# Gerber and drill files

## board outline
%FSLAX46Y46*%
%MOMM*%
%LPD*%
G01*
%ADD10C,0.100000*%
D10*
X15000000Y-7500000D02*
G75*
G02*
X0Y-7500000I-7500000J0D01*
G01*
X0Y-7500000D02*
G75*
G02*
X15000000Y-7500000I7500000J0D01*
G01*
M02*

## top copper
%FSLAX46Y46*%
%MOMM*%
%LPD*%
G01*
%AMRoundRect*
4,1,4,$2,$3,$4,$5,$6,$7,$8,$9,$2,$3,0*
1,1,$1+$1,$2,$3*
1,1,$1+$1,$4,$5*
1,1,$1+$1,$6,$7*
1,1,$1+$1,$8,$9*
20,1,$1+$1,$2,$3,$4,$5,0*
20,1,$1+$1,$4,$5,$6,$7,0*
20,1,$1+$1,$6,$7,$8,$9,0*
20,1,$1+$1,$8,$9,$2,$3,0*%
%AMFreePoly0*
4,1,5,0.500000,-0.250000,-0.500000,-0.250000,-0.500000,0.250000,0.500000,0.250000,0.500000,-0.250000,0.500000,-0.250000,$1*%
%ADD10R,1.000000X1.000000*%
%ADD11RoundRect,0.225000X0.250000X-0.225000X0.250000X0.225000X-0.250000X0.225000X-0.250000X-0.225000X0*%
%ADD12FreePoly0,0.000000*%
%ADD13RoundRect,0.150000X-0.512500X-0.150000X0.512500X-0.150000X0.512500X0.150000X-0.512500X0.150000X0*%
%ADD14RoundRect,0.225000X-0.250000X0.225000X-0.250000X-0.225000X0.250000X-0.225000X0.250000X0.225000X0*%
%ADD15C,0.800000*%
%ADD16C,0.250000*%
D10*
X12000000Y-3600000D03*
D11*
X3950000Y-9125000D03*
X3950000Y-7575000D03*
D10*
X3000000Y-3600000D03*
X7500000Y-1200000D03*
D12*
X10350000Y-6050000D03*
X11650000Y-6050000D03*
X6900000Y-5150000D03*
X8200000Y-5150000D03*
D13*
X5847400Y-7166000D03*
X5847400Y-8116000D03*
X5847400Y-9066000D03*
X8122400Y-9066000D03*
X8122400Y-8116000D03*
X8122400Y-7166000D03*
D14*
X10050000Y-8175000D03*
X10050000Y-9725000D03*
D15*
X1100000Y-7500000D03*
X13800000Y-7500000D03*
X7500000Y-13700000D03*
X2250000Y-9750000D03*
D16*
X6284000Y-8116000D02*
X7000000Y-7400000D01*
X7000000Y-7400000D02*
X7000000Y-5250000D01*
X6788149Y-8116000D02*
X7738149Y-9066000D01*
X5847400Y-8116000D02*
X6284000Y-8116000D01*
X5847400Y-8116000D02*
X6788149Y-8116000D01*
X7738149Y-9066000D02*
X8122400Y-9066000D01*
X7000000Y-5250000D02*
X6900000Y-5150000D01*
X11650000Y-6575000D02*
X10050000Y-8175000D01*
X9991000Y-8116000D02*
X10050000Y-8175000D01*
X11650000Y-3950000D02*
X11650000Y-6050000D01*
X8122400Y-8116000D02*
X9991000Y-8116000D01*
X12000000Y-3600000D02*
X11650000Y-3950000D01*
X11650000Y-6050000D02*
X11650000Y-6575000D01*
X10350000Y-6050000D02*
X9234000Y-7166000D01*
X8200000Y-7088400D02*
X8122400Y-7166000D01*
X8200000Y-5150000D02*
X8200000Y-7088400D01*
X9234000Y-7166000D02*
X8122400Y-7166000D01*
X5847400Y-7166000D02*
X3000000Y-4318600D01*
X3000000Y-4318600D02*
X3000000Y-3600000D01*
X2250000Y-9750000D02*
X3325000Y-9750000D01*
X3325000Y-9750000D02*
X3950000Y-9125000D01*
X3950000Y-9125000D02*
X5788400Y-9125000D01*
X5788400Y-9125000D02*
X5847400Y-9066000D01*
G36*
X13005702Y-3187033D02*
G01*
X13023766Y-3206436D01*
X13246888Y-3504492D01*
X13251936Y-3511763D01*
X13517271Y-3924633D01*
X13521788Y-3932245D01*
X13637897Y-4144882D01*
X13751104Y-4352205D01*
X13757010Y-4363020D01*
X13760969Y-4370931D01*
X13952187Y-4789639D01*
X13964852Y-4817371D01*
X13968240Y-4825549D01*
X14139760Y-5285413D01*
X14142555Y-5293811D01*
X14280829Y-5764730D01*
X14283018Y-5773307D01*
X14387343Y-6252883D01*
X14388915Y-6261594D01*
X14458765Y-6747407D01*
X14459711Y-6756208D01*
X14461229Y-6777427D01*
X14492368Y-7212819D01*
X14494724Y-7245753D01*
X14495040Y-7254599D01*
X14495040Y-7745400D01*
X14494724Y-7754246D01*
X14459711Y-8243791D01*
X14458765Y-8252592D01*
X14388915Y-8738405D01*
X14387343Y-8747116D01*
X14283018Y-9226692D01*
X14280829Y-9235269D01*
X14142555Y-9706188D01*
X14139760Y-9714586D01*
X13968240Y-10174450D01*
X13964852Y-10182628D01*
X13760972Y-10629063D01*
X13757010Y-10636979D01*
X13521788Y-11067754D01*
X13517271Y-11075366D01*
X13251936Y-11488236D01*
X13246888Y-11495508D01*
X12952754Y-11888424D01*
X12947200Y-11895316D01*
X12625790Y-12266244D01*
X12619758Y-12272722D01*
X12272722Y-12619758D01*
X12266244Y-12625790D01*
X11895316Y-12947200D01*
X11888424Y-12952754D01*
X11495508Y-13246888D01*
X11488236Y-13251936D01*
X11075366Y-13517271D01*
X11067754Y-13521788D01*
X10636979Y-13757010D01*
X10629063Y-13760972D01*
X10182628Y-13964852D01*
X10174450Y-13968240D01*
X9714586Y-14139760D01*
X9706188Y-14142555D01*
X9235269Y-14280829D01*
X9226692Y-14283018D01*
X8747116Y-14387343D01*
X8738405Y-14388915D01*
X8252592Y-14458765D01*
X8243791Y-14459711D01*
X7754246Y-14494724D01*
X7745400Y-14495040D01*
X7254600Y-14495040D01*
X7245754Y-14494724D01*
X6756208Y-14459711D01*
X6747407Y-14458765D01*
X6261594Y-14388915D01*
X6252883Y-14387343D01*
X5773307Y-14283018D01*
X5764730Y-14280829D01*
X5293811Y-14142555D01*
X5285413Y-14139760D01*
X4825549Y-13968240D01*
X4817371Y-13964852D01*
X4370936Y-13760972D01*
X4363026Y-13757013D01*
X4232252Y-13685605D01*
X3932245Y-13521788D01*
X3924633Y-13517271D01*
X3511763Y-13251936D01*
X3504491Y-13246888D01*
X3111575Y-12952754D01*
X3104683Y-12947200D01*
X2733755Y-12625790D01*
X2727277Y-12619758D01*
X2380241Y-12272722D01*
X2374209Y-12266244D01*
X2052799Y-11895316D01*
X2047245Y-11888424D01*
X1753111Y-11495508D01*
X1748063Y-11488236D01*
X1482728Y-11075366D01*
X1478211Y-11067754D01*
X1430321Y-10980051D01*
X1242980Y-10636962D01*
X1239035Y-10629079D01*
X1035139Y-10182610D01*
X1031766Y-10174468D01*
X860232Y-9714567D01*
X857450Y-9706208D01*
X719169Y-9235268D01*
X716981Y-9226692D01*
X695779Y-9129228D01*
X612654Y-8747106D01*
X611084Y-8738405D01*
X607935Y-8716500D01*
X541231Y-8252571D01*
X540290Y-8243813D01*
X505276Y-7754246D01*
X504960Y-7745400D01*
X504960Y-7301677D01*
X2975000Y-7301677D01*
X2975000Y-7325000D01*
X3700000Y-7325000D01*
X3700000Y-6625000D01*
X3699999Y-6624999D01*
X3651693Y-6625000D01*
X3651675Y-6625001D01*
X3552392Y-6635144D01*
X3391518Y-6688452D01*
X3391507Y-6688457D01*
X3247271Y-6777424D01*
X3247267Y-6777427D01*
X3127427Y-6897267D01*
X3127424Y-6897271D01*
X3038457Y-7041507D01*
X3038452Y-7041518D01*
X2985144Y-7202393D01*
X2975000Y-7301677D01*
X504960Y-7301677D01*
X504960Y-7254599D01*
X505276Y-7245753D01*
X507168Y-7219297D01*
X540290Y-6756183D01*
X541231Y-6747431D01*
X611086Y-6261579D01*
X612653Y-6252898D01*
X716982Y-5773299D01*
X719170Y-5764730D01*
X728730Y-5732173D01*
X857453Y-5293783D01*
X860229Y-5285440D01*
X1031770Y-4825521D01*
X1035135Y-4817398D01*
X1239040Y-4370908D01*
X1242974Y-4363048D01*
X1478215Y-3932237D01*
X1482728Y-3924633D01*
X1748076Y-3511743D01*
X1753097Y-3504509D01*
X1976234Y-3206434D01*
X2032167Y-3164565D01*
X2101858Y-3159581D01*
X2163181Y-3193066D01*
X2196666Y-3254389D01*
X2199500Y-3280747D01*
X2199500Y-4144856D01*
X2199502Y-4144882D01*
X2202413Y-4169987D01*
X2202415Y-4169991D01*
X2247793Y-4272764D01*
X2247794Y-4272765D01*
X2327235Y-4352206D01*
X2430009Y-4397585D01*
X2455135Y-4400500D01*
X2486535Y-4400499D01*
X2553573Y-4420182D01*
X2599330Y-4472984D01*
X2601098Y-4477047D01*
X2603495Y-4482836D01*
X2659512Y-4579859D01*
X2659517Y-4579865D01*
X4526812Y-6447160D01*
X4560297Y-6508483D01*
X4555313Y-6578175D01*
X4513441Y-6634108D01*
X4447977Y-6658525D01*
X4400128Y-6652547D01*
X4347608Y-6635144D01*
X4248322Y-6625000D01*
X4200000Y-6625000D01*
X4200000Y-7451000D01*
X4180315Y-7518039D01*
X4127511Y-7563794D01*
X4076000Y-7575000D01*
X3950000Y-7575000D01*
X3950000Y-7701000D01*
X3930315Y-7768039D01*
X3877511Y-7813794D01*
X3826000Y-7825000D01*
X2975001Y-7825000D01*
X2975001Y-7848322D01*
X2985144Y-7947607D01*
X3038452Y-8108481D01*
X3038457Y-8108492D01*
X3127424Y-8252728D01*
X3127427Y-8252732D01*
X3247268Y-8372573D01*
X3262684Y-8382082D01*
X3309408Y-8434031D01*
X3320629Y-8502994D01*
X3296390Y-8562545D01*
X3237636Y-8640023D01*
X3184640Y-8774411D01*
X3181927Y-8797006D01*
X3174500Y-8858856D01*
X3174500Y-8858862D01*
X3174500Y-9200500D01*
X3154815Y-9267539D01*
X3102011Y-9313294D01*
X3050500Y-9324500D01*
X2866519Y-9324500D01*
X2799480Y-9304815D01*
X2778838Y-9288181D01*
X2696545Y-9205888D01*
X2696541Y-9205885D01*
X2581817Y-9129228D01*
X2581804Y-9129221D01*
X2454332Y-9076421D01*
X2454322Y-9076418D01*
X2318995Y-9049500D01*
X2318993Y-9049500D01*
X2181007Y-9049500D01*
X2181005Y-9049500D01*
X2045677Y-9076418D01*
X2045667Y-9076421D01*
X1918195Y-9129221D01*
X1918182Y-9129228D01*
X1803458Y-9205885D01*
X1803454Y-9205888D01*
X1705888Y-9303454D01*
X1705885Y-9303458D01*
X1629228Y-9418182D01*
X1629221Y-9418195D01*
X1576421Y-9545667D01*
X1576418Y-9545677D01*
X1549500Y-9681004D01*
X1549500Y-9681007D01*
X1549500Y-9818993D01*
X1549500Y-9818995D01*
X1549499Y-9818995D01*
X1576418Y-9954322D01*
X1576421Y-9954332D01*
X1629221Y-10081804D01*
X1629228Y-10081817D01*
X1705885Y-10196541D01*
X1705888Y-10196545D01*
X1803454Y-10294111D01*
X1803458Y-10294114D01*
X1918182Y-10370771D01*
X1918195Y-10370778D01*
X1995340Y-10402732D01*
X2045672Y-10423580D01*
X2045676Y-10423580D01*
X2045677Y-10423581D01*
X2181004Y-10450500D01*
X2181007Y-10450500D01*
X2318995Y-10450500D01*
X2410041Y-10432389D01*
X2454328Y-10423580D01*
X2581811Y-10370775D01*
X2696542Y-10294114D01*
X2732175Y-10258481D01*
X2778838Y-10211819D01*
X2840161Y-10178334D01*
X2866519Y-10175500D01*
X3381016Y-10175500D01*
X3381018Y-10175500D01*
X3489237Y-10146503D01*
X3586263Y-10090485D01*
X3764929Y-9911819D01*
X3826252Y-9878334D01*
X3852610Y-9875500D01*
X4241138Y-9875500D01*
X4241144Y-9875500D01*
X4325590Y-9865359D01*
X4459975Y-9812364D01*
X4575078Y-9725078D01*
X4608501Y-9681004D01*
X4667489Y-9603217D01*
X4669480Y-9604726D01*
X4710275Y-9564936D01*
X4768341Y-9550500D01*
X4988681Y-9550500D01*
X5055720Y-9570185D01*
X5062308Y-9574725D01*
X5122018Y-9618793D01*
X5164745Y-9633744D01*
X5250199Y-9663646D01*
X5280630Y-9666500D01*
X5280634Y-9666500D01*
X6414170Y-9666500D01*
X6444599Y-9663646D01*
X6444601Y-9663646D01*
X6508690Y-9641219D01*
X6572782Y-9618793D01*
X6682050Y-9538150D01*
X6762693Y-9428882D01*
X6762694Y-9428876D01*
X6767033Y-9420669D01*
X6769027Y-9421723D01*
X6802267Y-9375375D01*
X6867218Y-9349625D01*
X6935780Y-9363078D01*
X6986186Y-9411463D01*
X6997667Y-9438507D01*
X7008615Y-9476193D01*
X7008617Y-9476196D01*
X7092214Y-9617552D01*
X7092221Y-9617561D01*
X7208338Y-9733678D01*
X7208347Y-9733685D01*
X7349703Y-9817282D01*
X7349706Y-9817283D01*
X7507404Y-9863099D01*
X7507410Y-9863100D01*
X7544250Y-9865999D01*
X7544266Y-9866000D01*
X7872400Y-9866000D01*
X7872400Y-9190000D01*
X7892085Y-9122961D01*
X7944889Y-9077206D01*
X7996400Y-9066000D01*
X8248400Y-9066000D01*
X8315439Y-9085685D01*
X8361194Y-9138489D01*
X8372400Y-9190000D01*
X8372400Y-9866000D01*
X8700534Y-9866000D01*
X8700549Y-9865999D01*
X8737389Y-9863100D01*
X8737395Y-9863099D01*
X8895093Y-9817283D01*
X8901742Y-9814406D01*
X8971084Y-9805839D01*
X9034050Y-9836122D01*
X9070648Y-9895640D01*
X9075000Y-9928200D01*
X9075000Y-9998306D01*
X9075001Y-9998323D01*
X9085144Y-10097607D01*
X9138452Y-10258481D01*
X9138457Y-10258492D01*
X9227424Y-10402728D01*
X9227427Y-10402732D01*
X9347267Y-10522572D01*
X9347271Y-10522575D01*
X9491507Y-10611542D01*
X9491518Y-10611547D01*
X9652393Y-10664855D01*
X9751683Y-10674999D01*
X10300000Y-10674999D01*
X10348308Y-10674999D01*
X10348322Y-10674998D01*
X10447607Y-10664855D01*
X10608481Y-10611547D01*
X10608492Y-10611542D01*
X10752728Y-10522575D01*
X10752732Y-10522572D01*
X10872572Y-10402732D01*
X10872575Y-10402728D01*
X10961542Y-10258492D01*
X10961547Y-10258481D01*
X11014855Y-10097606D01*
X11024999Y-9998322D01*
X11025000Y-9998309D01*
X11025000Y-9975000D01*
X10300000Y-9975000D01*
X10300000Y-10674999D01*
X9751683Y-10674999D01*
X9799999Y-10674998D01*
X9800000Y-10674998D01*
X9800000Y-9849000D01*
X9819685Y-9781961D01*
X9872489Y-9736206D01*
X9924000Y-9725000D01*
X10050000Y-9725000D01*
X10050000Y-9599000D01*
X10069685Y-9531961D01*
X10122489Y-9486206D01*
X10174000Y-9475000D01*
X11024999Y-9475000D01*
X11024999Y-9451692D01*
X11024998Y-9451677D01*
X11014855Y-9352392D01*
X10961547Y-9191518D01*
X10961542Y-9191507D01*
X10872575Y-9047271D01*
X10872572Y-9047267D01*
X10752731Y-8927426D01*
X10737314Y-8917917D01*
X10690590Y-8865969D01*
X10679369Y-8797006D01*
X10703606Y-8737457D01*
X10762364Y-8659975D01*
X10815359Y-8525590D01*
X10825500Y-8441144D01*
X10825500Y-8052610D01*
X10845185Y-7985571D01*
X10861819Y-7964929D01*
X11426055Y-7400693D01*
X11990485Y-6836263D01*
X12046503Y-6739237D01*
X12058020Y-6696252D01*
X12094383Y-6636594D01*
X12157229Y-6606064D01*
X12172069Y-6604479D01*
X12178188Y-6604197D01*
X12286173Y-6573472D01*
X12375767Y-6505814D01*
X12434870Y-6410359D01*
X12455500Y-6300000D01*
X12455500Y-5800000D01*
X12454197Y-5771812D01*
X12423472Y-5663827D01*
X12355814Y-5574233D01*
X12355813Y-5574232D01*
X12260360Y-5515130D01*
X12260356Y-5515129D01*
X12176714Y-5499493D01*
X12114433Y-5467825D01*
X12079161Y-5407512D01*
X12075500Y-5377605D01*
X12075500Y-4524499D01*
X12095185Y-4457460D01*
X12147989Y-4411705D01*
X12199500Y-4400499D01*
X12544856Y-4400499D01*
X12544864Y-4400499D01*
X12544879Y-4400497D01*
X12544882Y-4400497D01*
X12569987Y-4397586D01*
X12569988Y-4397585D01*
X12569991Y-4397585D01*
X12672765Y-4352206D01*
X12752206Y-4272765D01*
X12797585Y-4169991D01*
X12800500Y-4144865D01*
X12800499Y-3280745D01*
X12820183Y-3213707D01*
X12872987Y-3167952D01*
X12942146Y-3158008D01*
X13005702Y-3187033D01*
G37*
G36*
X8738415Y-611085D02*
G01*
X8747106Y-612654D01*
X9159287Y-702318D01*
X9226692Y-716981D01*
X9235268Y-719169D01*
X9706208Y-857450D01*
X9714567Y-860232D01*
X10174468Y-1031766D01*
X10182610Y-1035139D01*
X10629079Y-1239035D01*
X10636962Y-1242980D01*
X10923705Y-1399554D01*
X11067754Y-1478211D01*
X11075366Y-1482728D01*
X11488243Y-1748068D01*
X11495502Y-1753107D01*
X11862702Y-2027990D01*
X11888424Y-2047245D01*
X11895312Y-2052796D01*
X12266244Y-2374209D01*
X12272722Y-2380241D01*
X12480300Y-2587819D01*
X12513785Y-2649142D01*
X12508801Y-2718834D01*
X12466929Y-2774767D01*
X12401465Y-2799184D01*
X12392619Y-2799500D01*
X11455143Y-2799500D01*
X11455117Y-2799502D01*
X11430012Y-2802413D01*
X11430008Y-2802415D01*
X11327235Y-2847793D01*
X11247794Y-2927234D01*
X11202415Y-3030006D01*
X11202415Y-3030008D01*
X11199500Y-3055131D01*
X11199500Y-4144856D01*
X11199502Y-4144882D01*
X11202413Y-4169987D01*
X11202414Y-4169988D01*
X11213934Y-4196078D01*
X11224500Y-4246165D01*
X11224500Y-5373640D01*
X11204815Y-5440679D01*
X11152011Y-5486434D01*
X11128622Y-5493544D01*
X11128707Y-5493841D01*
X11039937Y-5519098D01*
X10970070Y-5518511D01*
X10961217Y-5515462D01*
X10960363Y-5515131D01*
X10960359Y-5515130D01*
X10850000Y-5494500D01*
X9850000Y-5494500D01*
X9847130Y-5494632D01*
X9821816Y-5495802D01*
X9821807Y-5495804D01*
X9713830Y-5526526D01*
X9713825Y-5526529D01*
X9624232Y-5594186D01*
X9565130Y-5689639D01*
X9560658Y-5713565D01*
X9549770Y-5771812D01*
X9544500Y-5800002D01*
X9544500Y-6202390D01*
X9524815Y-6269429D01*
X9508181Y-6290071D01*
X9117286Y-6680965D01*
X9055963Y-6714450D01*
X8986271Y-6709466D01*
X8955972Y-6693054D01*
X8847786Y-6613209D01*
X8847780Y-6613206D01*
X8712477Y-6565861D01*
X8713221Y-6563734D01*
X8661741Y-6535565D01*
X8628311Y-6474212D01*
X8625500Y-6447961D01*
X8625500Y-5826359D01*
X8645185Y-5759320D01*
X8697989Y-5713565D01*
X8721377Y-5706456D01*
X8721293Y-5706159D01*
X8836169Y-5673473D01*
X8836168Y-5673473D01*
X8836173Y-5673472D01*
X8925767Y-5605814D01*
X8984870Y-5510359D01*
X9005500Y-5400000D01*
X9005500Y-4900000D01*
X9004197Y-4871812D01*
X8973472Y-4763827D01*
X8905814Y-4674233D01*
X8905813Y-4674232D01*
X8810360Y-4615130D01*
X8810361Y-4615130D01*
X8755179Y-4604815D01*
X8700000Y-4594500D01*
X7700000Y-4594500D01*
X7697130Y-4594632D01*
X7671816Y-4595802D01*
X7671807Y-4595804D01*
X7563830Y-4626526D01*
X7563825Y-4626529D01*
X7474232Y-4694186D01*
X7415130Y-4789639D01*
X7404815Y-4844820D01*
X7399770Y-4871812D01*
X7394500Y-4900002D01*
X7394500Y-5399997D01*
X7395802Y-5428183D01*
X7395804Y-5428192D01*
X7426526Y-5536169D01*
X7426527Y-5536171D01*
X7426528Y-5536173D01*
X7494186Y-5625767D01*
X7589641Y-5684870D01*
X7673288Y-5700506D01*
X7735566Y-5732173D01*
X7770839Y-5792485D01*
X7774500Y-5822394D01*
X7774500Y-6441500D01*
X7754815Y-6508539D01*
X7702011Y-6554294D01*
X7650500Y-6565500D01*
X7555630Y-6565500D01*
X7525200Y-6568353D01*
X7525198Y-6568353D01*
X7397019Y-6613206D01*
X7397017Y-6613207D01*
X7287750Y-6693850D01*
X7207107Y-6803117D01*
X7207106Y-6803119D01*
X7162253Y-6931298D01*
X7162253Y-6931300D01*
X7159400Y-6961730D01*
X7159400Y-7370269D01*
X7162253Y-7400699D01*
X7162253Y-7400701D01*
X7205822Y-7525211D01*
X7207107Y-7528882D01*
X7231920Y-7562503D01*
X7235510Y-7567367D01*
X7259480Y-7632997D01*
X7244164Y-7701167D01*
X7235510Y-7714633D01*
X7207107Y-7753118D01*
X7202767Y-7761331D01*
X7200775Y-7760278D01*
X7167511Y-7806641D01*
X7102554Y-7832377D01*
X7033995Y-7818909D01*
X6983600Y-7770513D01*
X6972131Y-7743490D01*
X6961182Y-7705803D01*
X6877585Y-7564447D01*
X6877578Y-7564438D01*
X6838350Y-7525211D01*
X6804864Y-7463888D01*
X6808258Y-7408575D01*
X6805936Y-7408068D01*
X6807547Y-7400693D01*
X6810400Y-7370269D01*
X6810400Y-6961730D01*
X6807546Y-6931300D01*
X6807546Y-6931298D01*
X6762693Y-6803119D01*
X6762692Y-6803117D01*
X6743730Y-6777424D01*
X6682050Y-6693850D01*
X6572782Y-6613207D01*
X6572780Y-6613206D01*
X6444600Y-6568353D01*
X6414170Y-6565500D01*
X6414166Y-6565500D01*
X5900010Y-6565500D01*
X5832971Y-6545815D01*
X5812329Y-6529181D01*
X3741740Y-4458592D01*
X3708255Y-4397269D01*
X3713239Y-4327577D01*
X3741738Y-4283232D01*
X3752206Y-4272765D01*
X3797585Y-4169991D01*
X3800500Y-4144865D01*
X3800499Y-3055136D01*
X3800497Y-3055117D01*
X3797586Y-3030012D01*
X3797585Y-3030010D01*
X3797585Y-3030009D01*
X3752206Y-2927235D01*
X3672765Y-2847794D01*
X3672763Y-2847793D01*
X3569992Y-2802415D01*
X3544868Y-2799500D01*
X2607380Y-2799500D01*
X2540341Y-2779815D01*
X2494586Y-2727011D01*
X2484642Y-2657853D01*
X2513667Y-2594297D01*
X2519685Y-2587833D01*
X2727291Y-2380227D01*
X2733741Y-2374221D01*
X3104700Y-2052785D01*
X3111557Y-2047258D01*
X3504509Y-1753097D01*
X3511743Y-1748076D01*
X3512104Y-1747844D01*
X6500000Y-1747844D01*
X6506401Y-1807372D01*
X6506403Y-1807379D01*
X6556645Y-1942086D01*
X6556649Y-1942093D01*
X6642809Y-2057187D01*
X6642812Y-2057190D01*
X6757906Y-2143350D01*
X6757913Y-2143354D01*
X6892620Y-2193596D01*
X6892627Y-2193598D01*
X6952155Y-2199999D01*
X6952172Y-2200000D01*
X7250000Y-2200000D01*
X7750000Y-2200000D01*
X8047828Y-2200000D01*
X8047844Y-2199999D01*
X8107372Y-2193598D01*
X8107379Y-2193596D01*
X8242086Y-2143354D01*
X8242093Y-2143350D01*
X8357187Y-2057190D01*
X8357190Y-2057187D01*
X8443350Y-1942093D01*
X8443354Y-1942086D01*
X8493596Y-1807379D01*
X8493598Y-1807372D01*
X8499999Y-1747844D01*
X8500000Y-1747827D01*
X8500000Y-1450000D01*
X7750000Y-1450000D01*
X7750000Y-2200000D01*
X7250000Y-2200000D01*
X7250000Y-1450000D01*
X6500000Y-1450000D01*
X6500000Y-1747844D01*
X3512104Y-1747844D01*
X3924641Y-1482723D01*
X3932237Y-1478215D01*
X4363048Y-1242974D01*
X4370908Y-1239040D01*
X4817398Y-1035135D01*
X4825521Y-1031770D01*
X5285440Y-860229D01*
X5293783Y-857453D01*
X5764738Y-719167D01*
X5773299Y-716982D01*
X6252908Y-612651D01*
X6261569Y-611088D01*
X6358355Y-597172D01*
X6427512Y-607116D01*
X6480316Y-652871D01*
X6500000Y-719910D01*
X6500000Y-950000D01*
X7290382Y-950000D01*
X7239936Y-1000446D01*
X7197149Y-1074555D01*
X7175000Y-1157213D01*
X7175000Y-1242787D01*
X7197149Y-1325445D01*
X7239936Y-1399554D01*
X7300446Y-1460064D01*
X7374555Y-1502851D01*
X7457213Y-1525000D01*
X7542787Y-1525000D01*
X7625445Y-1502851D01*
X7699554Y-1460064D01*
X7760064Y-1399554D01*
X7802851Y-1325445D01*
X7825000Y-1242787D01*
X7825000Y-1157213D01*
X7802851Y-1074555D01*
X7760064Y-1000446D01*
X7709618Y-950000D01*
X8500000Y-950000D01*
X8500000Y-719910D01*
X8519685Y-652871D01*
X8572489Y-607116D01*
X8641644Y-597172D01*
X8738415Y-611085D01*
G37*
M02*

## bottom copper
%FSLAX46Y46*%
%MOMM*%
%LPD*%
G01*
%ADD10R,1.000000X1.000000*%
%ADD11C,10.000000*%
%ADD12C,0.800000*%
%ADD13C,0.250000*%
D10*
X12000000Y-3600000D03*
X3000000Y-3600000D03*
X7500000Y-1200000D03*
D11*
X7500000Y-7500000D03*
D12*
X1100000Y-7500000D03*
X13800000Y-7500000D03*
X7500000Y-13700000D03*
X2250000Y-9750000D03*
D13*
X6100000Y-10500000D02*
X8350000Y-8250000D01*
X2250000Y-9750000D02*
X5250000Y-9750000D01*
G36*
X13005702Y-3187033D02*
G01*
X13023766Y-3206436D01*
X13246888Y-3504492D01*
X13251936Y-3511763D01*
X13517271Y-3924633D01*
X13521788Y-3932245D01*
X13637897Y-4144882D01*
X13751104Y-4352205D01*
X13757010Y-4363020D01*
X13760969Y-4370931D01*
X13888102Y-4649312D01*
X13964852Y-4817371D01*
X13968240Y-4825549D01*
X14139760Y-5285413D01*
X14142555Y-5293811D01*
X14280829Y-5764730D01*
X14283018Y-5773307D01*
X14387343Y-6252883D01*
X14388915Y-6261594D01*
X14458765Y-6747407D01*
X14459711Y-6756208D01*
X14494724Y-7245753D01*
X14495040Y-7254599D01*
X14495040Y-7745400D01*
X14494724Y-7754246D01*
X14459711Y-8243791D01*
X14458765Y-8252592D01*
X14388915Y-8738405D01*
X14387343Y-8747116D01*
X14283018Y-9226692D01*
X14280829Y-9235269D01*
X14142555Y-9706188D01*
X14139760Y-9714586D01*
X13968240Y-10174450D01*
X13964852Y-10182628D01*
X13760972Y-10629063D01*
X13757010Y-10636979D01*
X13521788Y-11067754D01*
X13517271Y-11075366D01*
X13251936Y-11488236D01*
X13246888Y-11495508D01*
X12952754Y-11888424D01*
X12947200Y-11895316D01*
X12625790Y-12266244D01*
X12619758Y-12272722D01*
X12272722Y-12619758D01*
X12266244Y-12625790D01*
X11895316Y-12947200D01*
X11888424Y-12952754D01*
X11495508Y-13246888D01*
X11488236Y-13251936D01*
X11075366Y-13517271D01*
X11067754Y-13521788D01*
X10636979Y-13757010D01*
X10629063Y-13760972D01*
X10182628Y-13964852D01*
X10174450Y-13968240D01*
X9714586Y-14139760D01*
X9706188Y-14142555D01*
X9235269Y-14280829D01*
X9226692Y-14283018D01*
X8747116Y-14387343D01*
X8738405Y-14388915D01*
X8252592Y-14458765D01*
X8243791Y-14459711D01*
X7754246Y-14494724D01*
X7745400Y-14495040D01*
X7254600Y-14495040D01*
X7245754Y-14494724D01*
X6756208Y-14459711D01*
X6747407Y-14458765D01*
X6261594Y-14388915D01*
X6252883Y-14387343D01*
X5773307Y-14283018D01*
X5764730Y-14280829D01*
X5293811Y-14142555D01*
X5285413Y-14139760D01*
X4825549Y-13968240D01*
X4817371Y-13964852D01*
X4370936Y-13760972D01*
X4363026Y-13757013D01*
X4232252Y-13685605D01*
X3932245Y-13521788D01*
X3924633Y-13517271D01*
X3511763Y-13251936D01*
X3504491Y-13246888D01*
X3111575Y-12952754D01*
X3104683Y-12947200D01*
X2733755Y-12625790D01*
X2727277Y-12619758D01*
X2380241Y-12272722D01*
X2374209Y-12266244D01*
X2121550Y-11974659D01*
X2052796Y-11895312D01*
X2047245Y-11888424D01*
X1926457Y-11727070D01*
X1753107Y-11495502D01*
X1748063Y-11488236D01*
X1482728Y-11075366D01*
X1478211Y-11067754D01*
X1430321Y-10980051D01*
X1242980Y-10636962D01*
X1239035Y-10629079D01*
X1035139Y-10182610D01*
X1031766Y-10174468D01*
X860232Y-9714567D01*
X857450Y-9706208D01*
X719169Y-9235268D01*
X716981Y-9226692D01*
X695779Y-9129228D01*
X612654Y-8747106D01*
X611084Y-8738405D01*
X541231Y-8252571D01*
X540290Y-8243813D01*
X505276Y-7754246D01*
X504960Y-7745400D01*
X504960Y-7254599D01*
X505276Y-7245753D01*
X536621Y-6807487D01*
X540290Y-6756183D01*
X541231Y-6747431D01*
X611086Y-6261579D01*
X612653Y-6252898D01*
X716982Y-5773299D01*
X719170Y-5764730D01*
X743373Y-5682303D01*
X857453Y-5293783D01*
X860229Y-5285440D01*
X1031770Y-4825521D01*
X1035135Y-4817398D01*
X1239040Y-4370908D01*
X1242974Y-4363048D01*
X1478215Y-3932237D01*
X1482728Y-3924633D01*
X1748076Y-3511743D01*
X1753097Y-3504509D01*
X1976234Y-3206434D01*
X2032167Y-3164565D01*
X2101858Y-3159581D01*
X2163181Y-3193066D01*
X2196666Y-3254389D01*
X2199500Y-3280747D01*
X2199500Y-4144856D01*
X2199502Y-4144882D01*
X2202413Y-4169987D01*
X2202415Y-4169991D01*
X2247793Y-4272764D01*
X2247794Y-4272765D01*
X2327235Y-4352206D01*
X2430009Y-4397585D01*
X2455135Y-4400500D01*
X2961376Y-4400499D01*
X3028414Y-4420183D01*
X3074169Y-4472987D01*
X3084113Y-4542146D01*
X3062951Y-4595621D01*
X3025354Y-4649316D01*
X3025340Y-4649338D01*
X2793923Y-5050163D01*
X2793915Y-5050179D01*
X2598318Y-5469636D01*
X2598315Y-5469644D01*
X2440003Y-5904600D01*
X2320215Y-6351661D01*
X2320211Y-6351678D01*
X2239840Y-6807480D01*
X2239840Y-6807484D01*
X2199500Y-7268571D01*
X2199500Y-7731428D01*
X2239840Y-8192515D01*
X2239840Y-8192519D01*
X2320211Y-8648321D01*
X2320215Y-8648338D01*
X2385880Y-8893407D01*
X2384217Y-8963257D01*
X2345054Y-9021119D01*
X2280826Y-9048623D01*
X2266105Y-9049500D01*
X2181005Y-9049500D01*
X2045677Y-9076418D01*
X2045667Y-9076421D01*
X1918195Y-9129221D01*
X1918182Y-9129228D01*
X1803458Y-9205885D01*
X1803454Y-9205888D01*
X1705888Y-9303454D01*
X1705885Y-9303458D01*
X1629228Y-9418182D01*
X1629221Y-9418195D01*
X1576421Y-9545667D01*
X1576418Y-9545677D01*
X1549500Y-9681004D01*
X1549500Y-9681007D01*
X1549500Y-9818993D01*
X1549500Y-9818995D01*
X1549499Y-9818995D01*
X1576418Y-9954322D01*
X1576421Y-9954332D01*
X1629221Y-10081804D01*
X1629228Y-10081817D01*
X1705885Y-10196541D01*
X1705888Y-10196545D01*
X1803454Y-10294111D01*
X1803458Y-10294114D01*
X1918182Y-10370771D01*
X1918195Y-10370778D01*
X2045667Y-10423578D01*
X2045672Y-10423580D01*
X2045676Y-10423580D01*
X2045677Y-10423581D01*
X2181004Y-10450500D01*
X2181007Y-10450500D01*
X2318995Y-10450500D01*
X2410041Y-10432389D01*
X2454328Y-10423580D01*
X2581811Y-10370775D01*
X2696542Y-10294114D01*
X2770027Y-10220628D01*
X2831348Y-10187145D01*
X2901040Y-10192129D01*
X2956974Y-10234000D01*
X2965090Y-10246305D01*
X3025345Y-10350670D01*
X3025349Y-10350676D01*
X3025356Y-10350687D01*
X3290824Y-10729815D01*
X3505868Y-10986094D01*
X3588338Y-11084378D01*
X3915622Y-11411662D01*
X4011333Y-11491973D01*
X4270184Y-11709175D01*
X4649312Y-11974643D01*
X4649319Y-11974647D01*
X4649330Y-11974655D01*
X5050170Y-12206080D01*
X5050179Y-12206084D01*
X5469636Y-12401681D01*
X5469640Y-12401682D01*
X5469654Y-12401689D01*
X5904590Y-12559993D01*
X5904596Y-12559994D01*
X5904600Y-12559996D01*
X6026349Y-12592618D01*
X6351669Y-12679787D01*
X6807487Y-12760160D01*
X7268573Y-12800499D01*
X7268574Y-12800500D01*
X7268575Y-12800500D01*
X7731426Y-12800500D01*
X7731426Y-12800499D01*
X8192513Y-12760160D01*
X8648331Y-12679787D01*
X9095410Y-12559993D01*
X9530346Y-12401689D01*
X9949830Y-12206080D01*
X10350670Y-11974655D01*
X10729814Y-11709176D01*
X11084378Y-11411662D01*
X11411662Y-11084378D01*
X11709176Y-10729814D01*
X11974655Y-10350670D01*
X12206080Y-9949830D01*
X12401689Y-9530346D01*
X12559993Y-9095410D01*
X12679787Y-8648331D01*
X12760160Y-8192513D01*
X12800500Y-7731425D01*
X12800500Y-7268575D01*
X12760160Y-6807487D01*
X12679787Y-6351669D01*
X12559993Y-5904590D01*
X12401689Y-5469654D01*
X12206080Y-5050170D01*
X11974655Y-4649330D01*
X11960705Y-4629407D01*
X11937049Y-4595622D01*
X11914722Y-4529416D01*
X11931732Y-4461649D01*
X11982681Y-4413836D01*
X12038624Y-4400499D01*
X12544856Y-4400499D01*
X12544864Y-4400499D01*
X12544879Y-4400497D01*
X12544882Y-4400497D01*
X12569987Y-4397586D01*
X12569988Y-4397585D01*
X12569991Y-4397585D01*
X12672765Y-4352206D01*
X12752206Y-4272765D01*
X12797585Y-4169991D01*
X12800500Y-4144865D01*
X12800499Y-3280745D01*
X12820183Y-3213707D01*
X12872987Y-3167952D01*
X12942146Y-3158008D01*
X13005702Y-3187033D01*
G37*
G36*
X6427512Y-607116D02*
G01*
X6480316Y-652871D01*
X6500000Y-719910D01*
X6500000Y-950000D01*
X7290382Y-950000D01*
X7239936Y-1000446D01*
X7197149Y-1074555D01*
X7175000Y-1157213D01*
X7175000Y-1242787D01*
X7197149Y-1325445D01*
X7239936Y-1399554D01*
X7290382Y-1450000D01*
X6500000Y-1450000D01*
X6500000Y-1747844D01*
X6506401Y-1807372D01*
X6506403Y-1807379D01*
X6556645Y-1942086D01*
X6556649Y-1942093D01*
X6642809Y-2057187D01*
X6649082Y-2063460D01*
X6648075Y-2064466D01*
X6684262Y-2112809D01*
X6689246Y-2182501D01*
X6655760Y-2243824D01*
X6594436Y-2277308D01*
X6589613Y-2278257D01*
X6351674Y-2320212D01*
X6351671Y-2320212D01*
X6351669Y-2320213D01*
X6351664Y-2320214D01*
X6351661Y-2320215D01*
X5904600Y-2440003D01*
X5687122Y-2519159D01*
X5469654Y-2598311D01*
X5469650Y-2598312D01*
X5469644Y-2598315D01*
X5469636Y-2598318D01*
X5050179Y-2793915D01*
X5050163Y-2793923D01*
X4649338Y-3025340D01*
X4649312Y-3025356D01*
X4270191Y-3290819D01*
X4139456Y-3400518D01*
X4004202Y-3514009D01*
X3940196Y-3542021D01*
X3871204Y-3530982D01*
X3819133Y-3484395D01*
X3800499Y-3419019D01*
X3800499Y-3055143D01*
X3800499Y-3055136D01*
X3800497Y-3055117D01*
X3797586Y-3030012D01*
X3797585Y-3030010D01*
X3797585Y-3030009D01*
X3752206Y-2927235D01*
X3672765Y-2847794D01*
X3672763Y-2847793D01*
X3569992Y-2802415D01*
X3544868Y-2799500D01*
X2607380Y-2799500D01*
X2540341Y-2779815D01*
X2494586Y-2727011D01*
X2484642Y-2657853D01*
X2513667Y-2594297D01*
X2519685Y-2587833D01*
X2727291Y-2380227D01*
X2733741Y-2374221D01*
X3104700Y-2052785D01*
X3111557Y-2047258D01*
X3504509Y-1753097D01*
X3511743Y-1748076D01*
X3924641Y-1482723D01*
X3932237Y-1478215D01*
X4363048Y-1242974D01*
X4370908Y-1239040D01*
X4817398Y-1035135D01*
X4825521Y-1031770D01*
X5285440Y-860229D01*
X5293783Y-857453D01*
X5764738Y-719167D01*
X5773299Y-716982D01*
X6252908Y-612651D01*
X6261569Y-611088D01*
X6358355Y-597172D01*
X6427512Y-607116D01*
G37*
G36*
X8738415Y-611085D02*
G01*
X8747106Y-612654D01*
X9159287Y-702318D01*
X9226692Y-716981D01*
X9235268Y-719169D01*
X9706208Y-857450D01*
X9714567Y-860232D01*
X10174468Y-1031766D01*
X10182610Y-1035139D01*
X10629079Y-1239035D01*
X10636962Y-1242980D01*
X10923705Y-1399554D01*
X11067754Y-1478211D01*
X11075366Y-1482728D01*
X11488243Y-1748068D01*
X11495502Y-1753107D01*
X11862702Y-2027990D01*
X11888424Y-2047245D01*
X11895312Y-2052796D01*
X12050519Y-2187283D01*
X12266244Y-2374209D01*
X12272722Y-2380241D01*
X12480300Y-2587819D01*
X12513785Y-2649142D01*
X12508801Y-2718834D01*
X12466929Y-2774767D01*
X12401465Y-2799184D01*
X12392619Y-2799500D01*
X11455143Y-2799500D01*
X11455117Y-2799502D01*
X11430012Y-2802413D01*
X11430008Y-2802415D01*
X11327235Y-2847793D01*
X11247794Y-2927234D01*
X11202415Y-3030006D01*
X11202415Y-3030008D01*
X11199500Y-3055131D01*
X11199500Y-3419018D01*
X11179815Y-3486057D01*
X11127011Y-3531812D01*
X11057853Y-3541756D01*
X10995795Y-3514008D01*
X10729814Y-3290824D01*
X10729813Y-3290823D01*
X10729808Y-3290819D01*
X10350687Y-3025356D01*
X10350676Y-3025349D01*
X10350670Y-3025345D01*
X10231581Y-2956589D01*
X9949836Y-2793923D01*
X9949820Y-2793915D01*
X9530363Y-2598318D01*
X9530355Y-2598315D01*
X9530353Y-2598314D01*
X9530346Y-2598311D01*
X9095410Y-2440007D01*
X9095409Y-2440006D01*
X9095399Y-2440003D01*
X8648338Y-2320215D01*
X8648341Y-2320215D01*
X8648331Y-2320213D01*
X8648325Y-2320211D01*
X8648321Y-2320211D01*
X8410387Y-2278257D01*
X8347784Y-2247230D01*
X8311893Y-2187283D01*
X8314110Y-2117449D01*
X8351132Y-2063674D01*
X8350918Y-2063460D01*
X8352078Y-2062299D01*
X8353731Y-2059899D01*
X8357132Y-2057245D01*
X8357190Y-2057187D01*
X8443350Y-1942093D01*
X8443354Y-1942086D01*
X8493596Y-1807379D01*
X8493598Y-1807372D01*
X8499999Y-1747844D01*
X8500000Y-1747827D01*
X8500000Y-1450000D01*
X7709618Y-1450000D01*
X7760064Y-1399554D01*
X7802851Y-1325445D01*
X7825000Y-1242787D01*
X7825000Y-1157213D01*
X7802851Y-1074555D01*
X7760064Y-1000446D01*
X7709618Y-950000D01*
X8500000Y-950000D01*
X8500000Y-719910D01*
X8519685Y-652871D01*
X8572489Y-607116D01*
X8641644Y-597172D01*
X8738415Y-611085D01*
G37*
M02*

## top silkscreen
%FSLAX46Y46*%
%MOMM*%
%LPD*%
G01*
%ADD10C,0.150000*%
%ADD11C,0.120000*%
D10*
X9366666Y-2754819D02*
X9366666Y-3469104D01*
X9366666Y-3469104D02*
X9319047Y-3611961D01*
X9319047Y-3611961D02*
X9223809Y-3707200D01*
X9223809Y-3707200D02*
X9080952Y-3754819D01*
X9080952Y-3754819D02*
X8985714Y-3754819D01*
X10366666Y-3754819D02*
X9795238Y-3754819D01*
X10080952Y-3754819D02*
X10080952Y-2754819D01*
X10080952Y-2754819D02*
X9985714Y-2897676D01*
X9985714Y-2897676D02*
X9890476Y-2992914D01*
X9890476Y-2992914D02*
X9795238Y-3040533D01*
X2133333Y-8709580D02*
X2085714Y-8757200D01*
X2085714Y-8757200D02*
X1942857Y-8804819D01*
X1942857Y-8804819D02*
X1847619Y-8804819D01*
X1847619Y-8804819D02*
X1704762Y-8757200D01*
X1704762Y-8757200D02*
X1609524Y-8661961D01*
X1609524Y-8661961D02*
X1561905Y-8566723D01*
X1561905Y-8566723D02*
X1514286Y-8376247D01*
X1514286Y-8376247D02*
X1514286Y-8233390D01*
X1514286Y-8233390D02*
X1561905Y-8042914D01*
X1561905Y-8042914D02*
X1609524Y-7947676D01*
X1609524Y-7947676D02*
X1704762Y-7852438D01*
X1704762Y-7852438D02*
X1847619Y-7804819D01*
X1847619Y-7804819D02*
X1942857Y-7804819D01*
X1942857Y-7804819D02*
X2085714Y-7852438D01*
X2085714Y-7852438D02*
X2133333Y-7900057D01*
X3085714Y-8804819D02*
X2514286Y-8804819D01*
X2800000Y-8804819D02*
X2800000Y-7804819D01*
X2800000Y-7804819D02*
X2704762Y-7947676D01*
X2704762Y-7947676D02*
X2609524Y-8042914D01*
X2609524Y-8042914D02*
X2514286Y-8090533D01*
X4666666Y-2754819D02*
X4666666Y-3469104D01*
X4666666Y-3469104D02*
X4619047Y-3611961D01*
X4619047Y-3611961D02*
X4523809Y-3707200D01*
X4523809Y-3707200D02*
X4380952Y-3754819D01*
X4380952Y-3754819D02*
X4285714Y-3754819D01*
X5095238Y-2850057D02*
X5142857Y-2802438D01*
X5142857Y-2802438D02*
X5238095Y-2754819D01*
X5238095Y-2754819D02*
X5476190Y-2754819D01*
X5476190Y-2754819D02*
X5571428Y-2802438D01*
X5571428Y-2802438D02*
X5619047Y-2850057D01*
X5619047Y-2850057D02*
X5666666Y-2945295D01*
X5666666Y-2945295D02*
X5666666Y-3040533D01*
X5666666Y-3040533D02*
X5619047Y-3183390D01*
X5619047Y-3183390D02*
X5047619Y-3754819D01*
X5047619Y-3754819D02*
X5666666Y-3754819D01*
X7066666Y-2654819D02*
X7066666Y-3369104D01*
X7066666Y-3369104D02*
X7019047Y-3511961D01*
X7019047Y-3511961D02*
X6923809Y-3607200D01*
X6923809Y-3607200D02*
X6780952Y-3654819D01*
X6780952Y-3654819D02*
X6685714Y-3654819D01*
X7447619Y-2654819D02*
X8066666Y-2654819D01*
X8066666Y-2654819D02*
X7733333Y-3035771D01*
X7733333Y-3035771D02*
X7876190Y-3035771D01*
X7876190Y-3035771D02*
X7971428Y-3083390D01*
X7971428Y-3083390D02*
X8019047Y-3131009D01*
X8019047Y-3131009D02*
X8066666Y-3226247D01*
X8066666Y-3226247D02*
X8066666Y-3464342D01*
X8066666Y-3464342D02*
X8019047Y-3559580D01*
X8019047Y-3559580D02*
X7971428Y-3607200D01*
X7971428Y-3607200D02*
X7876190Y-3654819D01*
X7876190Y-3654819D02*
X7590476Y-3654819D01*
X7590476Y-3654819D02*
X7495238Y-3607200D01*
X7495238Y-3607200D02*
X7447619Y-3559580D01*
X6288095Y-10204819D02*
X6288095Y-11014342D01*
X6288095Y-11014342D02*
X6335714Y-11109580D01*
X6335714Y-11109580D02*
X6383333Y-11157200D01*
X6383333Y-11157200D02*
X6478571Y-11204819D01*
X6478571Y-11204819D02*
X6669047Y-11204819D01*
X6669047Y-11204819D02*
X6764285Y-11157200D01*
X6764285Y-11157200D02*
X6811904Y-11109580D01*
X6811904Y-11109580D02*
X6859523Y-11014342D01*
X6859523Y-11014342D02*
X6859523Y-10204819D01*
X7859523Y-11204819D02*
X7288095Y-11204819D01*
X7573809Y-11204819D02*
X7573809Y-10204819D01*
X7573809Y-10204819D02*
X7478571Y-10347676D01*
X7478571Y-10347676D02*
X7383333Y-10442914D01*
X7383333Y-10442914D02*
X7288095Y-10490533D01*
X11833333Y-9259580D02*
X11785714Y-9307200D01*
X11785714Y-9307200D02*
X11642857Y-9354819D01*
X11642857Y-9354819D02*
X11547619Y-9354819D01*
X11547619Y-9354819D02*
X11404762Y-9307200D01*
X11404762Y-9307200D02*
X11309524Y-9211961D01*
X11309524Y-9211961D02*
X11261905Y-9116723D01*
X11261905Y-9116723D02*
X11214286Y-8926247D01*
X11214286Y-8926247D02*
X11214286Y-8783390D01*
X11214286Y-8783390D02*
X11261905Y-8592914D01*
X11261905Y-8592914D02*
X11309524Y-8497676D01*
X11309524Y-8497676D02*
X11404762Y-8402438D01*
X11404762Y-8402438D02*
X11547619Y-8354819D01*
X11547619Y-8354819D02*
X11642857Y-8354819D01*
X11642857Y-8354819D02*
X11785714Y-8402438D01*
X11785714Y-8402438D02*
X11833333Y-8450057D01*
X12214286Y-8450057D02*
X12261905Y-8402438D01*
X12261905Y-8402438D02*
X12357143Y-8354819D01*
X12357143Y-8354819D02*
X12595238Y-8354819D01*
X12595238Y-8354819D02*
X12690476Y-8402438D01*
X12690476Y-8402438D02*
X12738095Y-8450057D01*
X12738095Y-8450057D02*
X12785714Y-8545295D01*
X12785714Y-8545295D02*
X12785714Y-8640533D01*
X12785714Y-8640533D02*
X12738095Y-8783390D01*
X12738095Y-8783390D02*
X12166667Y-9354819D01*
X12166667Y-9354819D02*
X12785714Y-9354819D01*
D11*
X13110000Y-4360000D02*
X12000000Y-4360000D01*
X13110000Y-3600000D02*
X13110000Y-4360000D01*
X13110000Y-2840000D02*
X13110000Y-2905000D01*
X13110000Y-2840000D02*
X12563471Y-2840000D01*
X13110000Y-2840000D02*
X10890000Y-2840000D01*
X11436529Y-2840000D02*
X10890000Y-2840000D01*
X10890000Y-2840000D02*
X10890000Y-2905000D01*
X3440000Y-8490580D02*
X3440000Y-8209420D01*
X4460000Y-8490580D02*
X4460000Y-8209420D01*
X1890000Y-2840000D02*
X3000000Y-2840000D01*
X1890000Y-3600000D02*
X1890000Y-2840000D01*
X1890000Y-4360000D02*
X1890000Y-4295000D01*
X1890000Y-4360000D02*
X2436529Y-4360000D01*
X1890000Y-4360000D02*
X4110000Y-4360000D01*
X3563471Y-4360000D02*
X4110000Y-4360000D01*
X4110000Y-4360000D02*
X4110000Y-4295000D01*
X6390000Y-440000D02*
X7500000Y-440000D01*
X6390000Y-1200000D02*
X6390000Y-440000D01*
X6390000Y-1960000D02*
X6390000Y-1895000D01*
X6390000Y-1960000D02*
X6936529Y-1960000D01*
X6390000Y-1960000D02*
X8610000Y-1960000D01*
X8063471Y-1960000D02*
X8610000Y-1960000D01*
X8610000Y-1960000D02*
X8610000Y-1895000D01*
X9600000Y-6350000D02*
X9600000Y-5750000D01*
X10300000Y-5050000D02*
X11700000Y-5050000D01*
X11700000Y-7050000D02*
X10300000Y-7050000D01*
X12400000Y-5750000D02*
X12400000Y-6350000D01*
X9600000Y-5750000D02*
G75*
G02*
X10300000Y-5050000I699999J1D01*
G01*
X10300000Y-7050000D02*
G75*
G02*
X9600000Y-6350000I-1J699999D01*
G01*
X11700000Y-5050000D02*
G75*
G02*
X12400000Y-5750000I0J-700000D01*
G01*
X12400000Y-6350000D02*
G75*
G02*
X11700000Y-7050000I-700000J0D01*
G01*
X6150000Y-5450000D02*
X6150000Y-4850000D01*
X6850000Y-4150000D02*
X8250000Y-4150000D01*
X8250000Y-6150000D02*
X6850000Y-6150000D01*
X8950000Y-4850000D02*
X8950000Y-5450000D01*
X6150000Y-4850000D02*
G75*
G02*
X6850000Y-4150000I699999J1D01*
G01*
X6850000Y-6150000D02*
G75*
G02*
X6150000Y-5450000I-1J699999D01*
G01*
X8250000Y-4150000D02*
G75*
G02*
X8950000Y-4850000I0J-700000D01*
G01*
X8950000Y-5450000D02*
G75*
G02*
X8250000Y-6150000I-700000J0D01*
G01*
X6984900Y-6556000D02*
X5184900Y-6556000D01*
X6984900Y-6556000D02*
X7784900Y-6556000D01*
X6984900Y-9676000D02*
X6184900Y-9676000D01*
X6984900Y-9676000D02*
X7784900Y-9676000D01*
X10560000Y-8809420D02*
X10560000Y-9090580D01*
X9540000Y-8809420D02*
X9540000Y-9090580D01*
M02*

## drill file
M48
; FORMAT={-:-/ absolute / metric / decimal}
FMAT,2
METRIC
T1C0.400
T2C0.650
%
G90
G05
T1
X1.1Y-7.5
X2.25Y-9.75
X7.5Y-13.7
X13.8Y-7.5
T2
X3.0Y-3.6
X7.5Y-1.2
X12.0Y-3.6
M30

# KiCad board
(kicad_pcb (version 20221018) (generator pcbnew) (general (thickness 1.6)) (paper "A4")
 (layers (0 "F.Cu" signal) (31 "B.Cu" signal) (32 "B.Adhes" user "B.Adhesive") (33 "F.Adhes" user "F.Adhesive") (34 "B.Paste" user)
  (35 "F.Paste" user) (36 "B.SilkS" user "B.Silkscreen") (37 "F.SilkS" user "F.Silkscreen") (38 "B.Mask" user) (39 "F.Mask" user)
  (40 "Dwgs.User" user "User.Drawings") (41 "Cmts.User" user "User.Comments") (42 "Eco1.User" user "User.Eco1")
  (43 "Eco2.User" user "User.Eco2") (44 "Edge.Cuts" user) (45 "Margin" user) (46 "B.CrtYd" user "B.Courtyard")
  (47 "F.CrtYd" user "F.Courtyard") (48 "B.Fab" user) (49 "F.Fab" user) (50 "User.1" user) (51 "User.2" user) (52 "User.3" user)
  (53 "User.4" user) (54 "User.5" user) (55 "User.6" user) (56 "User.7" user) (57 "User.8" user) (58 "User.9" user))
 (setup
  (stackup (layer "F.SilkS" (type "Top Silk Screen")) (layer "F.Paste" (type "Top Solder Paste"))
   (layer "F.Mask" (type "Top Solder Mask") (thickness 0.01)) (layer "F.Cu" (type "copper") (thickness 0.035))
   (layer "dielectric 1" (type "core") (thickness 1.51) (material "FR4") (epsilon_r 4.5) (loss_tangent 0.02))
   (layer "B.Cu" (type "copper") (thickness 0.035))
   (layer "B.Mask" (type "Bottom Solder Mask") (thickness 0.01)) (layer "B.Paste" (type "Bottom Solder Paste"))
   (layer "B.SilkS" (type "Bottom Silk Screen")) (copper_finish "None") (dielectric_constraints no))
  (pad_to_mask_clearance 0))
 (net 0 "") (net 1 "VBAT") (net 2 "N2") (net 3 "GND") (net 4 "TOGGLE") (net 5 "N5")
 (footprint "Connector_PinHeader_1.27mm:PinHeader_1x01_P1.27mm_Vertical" (layer "F.Cu") (at 12 3.6 180)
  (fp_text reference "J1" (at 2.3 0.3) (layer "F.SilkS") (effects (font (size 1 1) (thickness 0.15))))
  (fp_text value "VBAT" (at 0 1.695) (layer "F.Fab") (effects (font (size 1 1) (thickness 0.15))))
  (fp_line (start -1.11 -0.76) (end 0 -0.76) (stroke (width 0.12) (type solid)) (layer "F.SilkS"))
  (fp_line (start -1.11 0) (end -1.11 -0.76) (stroke (width 0.12) (type solid)) (layer "F.SilkS"))
  (fp_line (start -1.11 0.76) (end -1.11 0.695) (stroke (width 0.12) (type solid)) (layer "F.SilkS"))
  (fp_line (start -1.11 0.76) (end -0.563471 0.76) (stroke (width 0.12) (type solid)) (layer "F.SilkS"))
  (fp_line (start -1.11 0.76) (end 1.11 0.76) (stroke (width 0.12) (type solid)) (layer "F.SilkS"))
  (fp_line (start 0.563471 0.76) (end 1.11 0.76) (stroke (width 0.12) (type solid)) (layer "F.SilkS"))
  (fp_line (start 1.11 0.76) (end 1.11 0.695) (stroke (width 0.12) (type solid)) (layer "F.SilkS"))
  (pad "1" thru_hole rect (at 0 0 180) (size 1 1) (drill 0.65) (layers "*.Cu" "*.Mask") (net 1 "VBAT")))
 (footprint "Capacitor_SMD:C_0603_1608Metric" (layer "F.Cu") (at 3.95 8.35 90)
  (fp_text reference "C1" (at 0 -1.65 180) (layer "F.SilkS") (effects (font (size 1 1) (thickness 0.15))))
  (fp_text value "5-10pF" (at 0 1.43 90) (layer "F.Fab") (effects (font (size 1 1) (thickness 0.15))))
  (fp_line (start -0.14058 -0.51) (end 0.14058 -0.51) (stroke (width 0.12) (type solid)) (layer "F.SilkS"))
  (fp_line (start -0.14058 0.51) (end 0.14058 0.51) (stroke (width 0.12) (type solid)) (layer "F.SilkS"))
  (pad "1" smd roundrect (at -0.775 0 90) (size 0.9 0.95) (layers "F.Cu" "F.Paste" "F.Mask") (roundrect_rratio 0.25) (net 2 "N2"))
  (pad "2" smd roundrect (at 0.775 0 90) (size 0.9 0.95) (layers "F.Cu" "F.Paste" "F.Mask") (roundrect_rratio 0.25) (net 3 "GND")))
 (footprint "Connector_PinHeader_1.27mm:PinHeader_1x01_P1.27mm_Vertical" (layer "F.Cu") (at 3 3.6)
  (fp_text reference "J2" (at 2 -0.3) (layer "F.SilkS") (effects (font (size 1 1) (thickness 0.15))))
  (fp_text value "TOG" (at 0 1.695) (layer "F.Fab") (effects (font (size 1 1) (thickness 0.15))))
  (fp_line (start -1.11 -0.76) (end 0 -0.76) (stroke (width 0.12) (type solid)) (layer "F.SilkS"))
  (fp_line (start -1.11 0) (end -1.11 -0.76) (stroke (width 0.12) (type solid)) (layer "F.SilkS"))
  (fp_line (start -1.11 0.76) (end -1.11 0.695) (stroke (width 0.12) (type solid)) (layer "F.SilkS"))
  (fp_line (start -1.11 0.76) (end -0.563471 0.76) (stroke (width 0.12) (type solid)) (layer "F.SilkS"))
  (fp_line (start -1.11 0.76) (end 1.11 0.76) (stroke (width 0.12) (type solid)) (layer "F.SilkS"))
  (fp_line (start 0.563471 0.76) (end 1.11 0.76) (stroke (width 0.12) (type solid)) (layer "F.SilkS"))
  (fp_line (start 1.11 0.76) (end 1.11 0.695) (stroke (width 0.12) (type solid)) (layer "F.SilkS"))
  (pad "1" thru_hole rect (at 0 0) (size 1 1) (drill 0.65) (layers "*.Cu" "*.Mask") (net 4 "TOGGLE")))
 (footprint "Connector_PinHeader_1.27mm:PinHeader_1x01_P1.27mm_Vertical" (layer "F.Cu") (at 7.5 1.2)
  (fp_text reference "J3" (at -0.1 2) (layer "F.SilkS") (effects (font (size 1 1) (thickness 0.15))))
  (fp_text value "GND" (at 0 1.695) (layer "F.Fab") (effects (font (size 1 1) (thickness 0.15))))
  (fp_line (start -1.11 -0.76) (end 0 -0.76) (stroke (width 0.12) (type solid)) (layer "F.SilkS"))
  (fp_line (start -1.11 0) (end -1.11 -0.76) (stroke (width 0.12) (type solid)) (layer "F.SilkS"))
  (fp_line (start -1.11 0.76) (end -1.11 0.695) (stroke (width 0.12) (type solid)) (layer "F.SilkS"))
  (fp_line (start -1.11 0.76) (end -0.563471 0.76) (stroke (width 0.12) (type solid)) (layer "F.SilkS"))
  (fp_line (start -1.11 0.76) (end 1.11 0.76) (stroke (width 0.12) (type solid)) (layer "F.SilkS"))
  (fp_line (start 0.563471 0.76) (end 1.11 0.76) (stroke (width 0.12) (type solid)) (layer "F.SilkS"))
  (fp_line (start 1.11 0.76) (end 1.11 0.695) (stroke (width 0.12) (type solid)) (layer "F.SilkS"))
  (pad "1" thru_hole rect (at 0 0) (size 1 1) (drill 0.65) (layers "*.Cu" "*.Mask") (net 3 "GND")))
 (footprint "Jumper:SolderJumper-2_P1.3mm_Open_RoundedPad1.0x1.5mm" (layer "F.Cu") (at 11 6.05)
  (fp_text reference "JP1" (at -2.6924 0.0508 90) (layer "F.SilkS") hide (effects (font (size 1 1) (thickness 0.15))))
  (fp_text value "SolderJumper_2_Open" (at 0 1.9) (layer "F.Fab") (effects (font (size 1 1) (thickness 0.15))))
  (fp_line (start -1.4 0.3) (end -1.4 -0.3) (stroke (width 0.12) (type solid)) (layer "F.SilkS"))
  (fp_line (start -0.7 -1) (end 0.7 -1) (stroke (width 0.12) (type solid)) (layer "F.SilkS"))
  (fp_line (start 0.7 1) (end -0.7 1) (stroke (width 0.12) (type solid)) (layer "F.SilkS"))
  (fp_line (start 1.4 -0.3) (end 1.4 0.3) (stroke (width 0.12) (type solid)) (layer "F.SilkS"))
  (fp_arc (start -1.4 -0.3) (mid -1.194975 -0.794975) (end -0.7 -1) (stroke (width 0.12) (type solid)) (layer "F.SilkS"))
  (fp_arc (start -0.7 1) (mid -1.194975 0.794975) (end -1.4 0.3) (stroke (width 0.12) (type solid)) (layer "F.SilkS"))
  (fp_arc (start 0.7 -1) (mid 1.194975 -0.794975) (end 1.4 -0.3) (stroke (width 0.12) (type solid)) (layer "F.SilkS"))
  (fp_arc (start 1.4 0.3) (mid 1.194975 0.794975) (end 0.7 1) (stroke (width 0.12) (type solid)) (layer "F.SilkS"))
  (pad "1" smd custom (at -0.65 0) (size 1 0.5) (layers "F.Cu" "F.Mask") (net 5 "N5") (zone_connect 2) (thermal_bridge_angle 45)
   (options (clearance outline) (anchor rect)) (primitives))
  (pad "2" smd custom (at 0.65 0) (size 1 0.5) (layers "F.Cu" "F.Mask") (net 1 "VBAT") (zone_connect 2) (thermal_bridge_angle 45)
   (options (clearance outline) (anchor rect)) (primitives)))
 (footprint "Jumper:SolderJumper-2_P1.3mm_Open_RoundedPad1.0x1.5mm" (layer "F.Cu") (at 7.55 5.15)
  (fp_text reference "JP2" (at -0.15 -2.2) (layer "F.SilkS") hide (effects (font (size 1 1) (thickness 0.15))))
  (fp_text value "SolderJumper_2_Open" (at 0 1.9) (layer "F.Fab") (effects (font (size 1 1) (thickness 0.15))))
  (fp_line (start -1.4 0.3) (end -1.4 -0.3) (stroke (width 0.12) (type solid)) (layer "F.SilkS"))
  (fp_line (start -0.7 -1) (end 0.7 -1) (stroke (width 0.12) (type solid)) (layer "F.SilkS"))
  (fp_line (start 0.7 1) (end -0.7 1) (stroke (width 0.12) (type solid)) (layer "F.SilkS"))
  (fp_line (start 1.4 -0.3) (end 1.4 0.3) (stroke (width 0.12) (type solid)) (layer "F.SilkS"))
  (fp_arc (start -1.4 -0.3) (mid -1.194975 -0.794975) (end -0.7 -1) (stroke (width 0.12) (type solid)) (layer "F.SilkS"))
  (fp_arc (start -0.7 1) (mid -1.194975 0.794975) (end -1.4 0.3) (stroke (width 0.12) (type solid)) (layer "F.SilkS"))
  (fp_arc (start 0.7 -1) (mid 1.194975 -0.794975) (end 1.4 -0.3) (stroke (width 0.12) (type solid)) (layer "F.SilkS"))
  (fp_arc (start 1.4 0.3) (mid 1.194975 0.794975) (end 0.7 1) (stroke (width 0.12) (type solid)) (layer "F.SilkS"))
  (pad "1" smd custom (at -0.65 0) (size 1 0.5) (layers "F.Cu" "F.Mask") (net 3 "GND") (zone_connect 2) (thermal_bridge_angle 45)
   (options (clearance outline) (anchor rect)) (primitives))
  (pad "2" smd custom (at 0.65 0) (size 1 0.5) (layers "F.Cu" "F.Mask") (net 5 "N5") (zone_connect 2) (thermal_bridge_angle 45)
   (options (clearance outline) (anchor rect)) (primitives)))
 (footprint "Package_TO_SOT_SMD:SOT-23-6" (layer "F.Cu") (at 6.9849 8.116)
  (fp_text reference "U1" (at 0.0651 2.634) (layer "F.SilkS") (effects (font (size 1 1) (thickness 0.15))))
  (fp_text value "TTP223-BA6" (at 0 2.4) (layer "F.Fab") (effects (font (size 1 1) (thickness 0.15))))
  (fp_line (start 0 -1.56) (end -1.8 -1.56) (stroke (width 0.12) (type solid)) (layer "F.SilkS"))
  (fp_line (start 0 -1.56) (end 0.8 -1.56) (stroke (width 0.12) (type solid)) (layer "F.SilkS"))
  (fp_line (start 0 1.56) (end -0.8 1.56) (stroke (width 0.12) (type solid)) (layer "F.SilkS"))
  (fp_line (start 0 1.56) (end 0.8 1.56) (stroke (width 0.12) (type solid)) (layer "F.SilkS"))
  (pad "1" smd roundrect (at -1.1375 -0.95) (size 1.325 0.6) (layers "F.Cu" "F.Paste" "F.Mask") (roundrect_rratio 0.25) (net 4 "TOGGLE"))
  (pad "2" smd roundrect (at -1.1375 0) (size 1.325 0.6) (layers "F.Cu" "F.Paste" "F.Mask") (roundrect_rratio 0.25) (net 3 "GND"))
  (pad "3" smd roundrect (at -1.1375 0.95) (size 1.325 0.6) (layers "F.Cu" "F.Paste" "F.Mask") (roundrect_rratio 0.25) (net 2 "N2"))
  (pad "4" smd roundrect (at 1.1375 0.95) (size 1.325 0.6) (layers "F.Cu" "F.Paste" "F.Mask") (roundrect_rratio 0.25) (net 3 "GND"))
  (pad "5" smd roundrect (at 1.1375 0) (size 1.325 0.6) (layers "F.Cu" "F.Paste" "F.Mask") (roundrect_rratio 0.25) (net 1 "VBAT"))
  (pad "6" smd roundrect (at 1.1375 -0.95) (size 1.325 0.6) (layers "F.Cu" "F.Paste" "F.Mask") (roundrect_rratio 0.25) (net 5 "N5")))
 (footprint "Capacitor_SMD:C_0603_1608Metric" (layer "F.Cu") (at 10.05 8.95 -90)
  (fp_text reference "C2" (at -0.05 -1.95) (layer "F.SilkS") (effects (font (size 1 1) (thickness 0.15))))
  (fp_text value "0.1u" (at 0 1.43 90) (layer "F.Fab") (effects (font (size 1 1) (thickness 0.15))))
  (fp_line (start -0.14058 -0.51) (end 0.14058 -0.51) (stroke (width 0.12) (type solid)) (layer "F.SilkS"))
  (fp_line (start -0.14058 0.51) (end 0.14058 0.51) (stroke (width 0.12) (type solid)) (layer "F.SilkS"))
  (pad "1" smd roundrect (at -0.775 0 270) (size 0.9 0.95) (layers "F.Cu" "F.Paste" "F.Mask") (roundrect_rratio 0.25) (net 1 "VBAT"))
  (pad "2" smd roundrect (at 0.775 0 270) (size 0.9 0.95) (layers "F.Cu" "F.Paste" "F.Mask") (roundrect_rratio 0.25) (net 3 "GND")))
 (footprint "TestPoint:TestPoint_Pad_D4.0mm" (layer "B.Cu") (at 7.5 7.5 180)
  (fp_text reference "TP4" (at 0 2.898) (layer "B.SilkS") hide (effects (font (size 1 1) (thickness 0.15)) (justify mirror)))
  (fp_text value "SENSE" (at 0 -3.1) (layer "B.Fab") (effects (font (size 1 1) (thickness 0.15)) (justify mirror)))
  (pad "1" smd circle (at 0 0 180) (size 10 10) (layers "B.Cu" "B.Mask") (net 2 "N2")))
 (gr_circle (center 7.5 7.5) (end 15 7.5) (stroke (width 0.1) (type default)) (fill none) (layer "Edge.Cuts"))
 (segment (start 6.284 8.116) (end 7 7.4) (width 0.25) (layer "F.Cu") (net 3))
 (segment (start 7 7.4) (end 7 5.25) (width 0.25) (layer "F.Cu") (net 3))
 (segment (start 6.788149 8.116) (end 7.738149 9.066) (width 0.25) (layer "F.Cu") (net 3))
 (segment (start 5.8474 8.116) (end 6.284 8.116) (width 0.25) (layer "F.Cu") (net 3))
 (segment (start 5.8474 8.116) (end 6.788149 8.116) (width 0.25) (layer "F.Cu") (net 3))
 (segment (start 7.738149 9.066) (end 8.1224 9.066) (width 0.25) (layer "F.Cu") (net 3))
 (segment (start 7 5.25) (end 6.9 5.15) (width 0.25) (layer "F.Cu") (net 3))
 (via (at 1.1 7.5) (size 0.8) (drill 0.4) (layers "F.Cu" "B.Cu") (free) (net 3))
 (via (at 13.8 7.5) (size 0.8) (drill 0.4) (layers "F.Cu" "B.Cu") (free) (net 3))
 (via (at 7.5 13.7) (size 0.8) (drill 0.4) (layers "F.Cu" "B.Cu") (free) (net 3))
 (segment (start 11.65 6.575) (end 10.05 8.175) (width 0.25) (layer "F.Cu") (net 1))
 (segment (start 9.991 8.116) (end 10.05 8.175) (width 0.25) (layer "F.Cu") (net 1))
 (segment (start 11.65 3.95) (end 11.65 6.05) (width 0.25) (layer "F.Cu") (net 1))
 (segment (start 8.1224 8.116) (end 9.991 8.116) (width 0.25) (layer "F.Cu") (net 1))
 (segment (start 12 3.6) (end 11.65 3.95) (width 0.25) (layer "F.Cu") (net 1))
 (segment (start 11.65 6.05) (end 11.65 6.575) (width 0.25) (layer "F.Cu") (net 1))
 (segment (start 10.35 6.05) (end 9.234 7.166) (width 0.25) (layer "F.Cu") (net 5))
 (segment (start 8.2 7.0884) (end 8.1224 7.166) (width 0.25) (layer "F.Cu") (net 5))
 (segment (start 8.2 5.15) (end 8.2 7.0884) (width 0.25) (layer "F.Cu") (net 5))
 (segment (start 9.234 7.166) (end 8.1224 7.166) (width 0.25) (layer "F.Cu") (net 5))
 (segment (start 5.8474 7.166) (end 3 4.3186) (width 0.25) (layer "F.Cu") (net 4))
 (segment (start 3 4.3186) (end 3 3.6) (width 0.25) (layer "F.Cu") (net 4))
 (segment (start 2.25 9.75) (end 3.325 9.75) (width 0.25) (layer "F.Cu") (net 2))
 (segment (start 3.325 9.75) (end 3.95 9.125) (width 0.25) (layer "F.Cu") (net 2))
 (segment (start 3.95 9.125) (end 5.7884 9.125) (width 0.25) (layer "F.Cu") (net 2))
 (segment (start 5.7884 9.125) (end 5.8474 9.066) (width 0.25) (layer "F.Cu") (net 2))
 (via (at 2.25 9.75) (size 0.8) (drill 0.4) (layers "F.Cu" "B.Cu") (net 2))
 (segment (start 6.1 10.5) (end 8.35 8.25) (width 0.25) (layer "B.Cu") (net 2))
 (segment (start 2.25 9.75) (end 5.25 9.75) (width 0.25) (layer "B.Cu") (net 2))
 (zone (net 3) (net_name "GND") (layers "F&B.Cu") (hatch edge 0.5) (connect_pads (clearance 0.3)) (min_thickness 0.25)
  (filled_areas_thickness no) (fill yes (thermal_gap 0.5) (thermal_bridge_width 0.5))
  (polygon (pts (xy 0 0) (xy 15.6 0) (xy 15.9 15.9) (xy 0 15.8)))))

